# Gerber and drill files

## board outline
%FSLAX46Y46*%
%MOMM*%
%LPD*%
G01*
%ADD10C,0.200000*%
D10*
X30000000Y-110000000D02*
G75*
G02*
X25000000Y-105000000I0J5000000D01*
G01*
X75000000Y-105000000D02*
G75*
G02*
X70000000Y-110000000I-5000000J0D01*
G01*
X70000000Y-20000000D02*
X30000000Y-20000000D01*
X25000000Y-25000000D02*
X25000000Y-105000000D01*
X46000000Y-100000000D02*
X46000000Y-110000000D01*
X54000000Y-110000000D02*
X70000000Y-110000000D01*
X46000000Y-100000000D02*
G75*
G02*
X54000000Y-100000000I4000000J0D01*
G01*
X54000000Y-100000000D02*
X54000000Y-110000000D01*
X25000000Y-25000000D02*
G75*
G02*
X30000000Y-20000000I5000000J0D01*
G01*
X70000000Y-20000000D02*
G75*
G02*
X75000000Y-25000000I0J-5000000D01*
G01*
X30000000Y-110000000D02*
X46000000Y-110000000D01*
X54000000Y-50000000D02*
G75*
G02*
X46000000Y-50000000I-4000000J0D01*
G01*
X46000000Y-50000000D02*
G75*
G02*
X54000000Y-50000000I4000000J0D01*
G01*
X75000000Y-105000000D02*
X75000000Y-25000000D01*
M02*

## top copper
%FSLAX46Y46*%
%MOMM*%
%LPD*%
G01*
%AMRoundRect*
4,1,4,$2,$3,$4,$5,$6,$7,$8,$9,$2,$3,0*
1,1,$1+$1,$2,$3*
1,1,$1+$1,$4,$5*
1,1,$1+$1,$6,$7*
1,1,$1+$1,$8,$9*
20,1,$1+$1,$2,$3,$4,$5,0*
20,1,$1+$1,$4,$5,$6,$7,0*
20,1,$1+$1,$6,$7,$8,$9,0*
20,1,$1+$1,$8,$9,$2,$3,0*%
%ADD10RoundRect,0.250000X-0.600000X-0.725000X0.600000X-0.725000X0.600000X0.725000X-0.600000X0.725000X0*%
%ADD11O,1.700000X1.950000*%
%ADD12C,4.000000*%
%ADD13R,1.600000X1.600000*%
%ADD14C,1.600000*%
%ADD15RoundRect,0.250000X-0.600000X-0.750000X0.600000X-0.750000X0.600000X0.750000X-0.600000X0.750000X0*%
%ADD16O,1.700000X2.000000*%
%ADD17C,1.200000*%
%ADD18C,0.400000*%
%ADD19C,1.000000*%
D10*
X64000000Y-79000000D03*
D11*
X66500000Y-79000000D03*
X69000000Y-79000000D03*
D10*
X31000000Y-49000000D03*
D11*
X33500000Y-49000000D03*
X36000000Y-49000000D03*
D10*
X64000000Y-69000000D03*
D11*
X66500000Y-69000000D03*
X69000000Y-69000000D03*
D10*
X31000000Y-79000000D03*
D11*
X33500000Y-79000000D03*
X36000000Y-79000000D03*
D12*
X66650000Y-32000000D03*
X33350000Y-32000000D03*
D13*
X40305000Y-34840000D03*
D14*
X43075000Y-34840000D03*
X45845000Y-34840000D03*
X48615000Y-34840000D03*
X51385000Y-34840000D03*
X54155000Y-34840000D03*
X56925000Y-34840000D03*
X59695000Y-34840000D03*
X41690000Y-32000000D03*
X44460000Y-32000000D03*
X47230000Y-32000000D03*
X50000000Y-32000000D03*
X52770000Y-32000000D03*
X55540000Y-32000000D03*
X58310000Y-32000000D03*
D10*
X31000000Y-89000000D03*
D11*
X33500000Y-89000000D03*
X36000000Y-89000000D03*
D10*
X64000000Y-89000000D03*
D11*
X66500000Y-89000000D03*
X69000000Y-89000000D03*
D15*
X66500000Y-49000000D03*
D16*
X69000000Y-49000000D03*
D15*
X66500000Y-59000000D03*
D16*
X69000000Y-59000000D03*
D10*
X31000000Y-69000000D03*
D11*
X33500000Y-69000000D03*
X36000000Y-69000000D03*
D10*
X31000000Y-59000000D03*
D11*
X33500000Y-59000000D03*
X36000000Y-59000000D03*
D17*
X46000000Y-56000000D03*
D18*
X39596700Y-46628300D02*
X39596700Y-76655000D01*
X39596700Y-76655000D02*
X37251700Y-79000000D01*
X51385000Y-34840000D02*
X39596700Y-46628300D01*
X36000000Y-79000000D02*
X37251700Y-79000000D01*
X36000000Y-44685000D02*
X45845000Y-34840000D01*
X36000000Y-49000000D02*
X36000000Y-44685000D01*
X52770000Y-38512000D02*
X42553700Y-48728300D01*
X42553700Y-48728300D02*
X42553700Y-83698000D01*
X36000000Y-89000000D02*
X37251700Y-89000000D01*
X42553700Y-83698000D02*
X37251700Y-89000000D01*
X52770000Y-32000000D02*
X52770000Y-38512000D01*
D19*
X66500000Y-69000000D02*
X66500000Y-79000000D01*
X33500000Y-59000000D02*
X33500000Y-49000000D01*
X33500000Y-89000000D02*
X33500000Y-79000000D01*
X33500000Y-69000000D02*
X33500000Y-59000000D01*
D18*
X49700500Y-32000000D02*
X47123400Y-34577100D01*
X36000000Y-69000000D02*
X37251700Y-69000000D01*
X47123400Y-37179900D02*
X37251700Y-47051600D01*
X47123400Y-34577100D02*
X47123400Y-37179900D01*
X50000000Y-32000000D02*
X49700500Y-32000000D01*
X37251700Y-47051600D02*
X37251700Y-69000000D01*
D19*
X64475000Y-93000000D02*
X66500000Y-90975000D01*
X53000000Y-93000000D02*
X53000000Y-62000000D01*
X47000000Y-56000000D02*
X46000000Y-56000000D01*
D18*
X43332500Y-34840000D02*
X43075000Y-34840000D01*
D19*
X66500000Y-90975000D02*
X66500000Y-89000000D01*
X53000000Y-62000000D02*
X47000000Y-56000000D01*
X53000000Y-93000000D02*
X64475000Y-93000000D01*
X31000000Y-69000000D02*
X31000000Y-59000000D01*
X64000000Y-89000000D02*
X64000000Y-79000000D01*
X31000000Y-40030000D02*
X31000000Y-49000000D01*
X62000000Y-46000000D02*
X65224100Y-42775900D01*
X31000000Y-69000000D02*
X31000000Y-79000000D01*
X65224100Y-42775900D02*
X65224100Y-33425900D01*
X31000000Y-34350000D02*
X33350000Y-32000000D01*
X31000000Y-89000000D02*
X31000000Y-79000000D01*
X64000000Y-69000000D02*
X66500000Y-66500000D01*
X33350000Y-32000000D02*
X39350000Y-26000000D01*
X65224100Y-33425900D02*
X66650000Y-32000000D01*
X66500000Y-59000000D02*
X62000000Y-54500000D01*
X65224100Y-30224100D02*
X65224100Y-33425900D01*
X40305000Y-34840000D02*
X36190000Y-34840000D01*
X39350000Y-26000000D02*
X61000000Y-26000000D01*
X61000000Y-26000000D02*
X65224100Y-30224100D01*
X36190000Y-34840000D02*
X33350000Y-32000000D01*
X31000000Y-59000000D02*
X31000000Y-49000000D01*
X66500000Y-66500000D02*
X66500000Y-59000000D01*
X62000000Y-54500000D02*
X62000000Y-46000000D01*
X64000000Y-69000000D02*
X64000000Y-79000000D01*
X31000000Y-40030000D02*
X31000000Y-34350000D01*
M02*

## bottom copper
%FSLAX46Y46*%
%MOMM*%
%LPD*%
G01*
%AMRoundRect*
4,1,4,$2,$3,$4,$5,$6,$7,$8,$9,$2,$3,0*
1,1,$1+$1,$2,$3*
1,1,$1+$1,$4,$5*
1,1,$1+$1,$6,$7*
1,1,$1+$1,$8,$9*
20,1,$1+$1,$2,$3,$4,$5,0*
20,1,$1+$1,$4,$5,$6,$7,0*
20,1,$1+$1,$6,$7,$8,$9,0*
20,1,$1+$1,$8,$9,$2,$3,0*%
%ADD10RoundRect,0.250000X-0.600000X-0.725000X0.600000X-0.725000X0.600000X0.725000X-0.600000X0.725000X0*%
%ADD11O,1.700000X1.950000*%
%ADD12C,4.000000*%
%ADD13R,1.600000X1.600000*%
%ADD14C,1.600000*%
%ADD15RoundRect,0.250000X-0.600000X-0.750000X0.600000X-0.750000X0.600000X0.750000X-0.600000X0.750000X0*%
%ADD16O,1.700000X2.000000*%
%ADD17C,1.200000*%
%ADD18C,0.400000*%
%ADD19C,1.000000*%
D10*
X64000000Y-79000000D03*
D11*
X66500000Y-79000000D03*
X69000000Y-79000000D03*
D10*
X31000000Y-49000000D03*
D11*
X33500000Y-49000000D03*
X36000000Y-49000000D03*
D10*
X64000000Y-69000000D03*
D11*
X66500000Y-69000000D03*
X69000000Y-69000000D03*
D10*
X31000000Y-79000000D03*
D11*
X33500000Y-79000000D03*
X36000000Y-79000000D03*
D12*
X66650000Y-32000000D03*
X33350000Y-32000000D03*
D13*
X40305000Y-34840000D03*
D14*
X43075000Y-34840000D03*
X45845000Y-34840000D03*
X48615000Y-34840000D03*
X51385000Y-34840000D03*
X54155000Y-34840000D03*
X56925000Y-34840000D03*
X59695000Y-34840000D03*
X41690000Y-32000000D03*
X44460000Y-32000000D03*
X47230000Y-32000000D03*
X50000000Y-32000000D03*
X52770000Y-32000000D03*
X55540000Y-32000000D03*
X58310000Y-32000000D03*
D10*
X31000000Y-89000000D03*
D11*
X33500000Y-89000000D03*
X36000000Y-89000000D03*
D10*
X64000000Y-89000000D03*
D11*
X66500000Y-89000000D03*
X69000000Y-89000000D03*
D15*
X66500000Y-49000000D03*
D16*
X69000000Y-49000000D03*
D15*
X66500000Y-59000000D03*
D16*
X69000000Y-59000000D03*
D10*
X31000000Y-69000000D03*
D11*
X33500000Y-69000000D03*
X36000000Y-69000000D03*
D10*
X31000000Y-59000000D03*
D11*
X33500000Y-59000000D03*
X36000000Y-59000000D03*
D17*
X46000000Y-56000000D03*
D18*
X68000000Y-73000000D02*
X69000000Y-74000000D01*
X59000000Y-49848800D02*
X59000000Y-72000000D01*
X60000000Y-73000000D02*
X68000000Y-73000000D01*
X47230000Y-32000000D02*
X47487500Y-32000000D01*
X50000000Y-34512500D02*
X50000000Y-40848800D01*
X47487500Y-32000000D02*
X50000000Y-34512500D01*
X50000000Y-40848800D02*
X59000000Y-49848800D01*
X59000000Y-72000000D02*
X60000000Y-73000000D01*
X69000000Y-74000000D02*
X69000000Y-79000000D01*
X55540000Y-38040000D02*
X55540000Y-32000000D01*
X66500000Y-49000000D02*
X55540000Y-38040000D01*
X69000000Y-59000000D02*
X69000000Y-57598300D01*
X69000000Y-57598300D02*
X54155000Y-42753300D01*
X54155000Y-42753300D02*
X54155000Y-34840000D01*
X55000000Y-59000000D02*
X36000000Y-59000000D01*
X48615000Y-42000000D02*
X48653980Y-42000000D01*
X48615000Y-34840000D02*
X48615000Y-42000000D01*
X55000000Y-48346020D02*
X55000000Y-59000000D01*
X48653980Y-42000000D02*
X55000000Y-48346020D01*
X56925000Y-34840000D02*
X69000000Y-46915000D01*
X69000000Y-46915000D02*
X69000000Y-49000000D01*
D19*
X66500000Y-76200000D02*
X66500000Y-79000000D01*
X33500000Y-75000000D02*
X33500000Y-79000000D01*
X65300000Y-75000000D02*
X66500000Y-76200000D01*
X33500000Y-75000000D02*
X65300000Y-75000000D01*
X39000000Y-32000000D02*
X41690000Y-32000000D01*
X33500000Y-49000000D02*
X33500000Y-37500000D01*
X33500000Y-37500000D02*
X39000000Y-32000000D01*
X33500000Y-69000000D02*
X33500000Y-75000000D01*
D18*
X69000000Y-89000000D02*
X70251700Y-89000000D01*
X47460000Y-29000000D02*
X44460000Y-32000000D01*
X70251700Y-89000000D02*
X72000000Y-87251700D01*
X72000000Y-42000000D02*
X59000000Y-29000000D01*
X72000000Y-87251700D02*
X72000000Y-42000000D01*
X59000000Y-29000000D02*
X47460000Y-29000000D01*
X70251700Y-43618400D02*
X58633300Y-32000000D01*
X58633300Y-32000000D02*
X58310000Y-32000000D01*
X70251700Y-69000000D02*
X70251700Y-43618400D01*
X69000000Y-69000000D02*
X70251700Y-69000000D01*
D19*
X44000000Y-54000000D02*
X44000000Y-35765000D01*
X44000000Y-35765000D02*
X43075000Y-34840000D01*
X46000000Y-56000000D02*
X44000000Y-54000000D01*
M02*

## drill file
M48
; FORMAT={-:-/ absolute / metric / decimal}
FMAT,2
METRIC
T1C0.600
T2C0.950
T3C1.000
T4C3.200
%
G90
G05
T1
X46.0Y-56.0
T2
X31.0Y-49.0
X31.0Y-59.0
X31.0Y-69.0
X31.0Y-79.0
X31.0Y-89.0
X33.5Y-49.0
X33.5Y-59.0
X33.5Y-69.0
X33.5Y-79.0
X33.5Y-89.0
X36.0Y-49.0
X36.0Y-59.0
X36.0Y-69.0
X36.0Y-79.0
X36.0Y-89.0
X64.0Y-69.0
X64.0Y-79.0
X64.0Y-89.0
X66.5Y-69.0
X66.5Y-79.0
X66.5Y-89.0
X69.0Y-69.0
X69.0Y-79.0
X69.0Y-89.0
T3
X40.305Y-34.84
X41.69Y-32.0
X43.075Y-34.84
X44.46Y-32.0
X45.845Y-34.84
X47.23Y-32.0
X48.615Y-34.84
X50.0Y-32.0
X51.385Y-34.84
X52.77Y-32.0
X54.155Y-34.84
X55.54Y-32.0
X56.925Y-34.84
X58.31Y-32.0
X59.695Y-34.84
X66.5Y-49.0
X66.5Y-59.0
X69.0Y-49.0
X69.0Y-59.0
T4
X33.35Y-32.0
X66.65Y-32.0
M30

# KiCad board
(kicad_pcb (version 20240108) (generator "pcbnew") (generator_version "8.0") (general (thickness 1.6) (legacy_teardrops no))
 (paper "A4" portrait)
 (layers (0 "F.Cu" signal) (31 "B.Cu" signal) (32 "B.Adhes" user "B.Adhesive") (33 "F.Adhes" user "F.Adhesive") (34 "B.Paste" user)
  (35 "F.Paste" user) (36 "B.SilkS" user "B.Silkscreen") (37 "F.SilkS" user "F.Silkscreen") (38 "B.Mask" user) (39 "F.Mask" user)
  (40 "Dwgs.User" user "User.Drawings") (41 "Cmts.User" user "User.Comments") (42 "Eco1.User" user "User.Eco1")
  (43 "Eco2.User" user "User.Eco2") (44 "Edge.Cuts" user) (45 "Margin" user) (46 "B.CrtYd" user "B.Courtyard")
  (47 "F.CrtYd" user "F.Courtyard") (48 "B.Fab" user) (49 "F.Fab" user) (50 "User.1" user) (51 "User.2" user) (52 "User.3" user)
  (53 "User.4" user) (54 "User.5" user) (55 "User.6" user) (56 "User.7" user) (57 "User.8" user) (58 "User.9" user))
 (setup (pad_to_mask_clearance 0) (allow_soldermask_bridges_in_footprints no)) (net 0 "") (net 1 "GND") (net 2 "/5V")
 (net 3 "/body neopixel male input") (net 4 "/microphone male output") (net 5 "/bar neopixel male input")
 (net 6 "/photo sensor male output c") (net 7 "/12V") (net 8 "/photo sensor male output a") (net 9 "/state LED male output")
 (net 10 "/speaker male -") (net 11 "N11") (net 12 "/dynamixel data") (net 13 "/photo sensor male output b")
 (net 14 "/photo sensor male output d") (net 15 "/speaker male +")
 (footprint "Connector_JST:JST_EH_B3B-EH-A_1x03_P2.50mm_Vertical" (layer "F.Cu") (at 64 79)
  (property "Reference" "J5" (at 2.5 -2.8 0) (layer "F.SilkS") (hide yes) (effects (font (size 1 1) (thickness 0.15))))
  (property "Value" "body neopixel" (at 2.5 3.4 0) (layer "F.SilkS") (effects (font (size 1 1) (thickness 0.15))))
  (pad "1" thru_hole roundrect (at 0 0) (size 1.7 1.95) (drill 0.95) (layers "*.Cu" "*.Mask") (remove_unused_layers no)
   (roundrect_rratio 0.147059) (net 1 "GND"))
  (pad "2" thru_hole oval (at 2.5 0) (size 1.7 1.95) (drill 0.95) (layers "*.Cu" "*.Mask") (remove_unused_layers no) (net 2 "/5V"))
  (pad "3" thru_hole oval (at 5 0) (size 1.7 1.95) (drill 0.95) (layers "*.Cu" "*.Mask") (remove_unused_layers no)
   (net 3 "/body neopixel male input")))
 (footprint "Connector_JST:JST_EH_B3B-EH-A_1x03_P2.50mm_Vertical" (layer "F.Cu") (at 31 49)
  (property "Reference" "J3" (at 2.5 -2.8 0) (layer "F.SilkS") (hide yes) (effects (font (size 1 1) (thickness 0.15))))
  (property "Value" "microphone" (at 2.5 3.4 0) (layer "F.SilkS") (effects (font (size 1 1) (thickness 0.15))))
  (pad "1" thru_hole roundrect (at 0 0) (size 1.7 1.95) (drill 0.95) (layers "*.Cu" "*.Mask") (remove_unused_layers no)
   (roundrect_rratio 0.147059) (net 1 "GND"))
  (pad "2" thru_hole oval (at 2.5 0) (size 1.7 1.95) (drill 0.95) (layers "*.Cu" "*.Mask") (remove_unused_layers no) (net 2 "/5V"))
  (pad "3" thru_hole oval (at 5 0) (size 1.7 1.95) (drill 0.95) (layers "*.Cu" "*.Mask") (remove_unused_layers no)
   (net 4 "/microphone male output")))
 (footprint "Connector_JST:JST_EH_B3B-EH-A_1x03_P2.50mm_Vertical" (layer "F.Cu") (at 64 69)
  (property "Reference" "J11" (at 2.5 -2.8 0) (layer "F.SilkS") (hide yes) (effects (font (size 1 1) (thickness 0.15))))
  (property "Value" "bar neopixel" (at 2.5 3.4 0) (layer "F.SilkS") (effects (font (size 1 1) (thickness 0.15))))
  (pad "1" thru_hole roundrect (at 0 0) (size 1.7 1.95) (drill 0.95) (layers "*.Cu" "*.Mask") (remove_unused_layers no)
   (roundrect_rratio 0.147059) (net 1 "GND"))
  (pad "2" thru_hole oval (at 2.5 0) (size 1.7 1.95) (drill 0.95) (layers "*.Cu" "*.Mask") (remove_unused_layers no) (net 2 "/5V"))
  (pad "3" thru_hole oval (at 5 0) (size 1.7 1.95) (drill 0.95) (layers "*.Cu" "*.Mask") (remove_unused_layers no)
   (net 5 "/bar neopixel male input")))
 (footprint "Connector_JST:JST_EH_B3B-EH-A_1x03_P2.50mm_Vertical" (layer "F.Cu") (at 31 79)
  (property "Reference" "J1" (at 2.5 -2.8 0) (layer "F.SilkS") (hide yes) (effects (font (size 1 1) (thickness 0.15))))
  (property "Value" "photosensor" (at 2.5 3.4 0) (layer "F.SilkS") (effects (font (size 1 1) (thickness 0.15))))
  (pad "1" thru_hole roundrect (at 0 0) (size 1.7 1.95) (drill 0.95) (layers "*.Cu" "*.Mask") (remove_unused_layers no)
   (roundrect_rratio 0.147059) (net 1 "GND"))
  (pad "2" thru_hole oval (at 2.5 0) (size 1.7 1.95) (drill 0.95) (layers "*.Cu" "*.Mask") (remove_unused_layers no) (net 2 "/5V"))
  (pad "3" thru_hole oval (at 5 0) (size 1.7 1.95) (drill 0.95) (layers "*.Cu" "*.Mask") (remove_unused_layers no)
   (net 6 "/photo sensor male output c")))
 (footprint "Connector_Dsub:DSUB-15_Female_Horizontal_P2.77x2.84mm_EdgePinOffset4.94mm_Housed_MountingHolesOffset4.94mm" (layer "F.Cu")
  (at 40.305 34.84 180)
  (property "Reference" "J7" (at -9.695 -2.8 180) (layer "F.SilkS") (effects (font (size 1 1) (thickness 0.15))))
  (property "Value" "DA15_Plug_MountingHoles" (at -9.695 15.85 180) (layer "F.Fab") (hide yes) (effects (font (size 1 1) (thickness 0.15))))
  (pad "0" thru_hole circle (at -26.345 2.84 180) (size 4 4) (drill 3.2) (layers "*.Cu" "*.Mask") (remove_unused_layers no) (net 1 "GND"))
  (pad "0" thru_hole circle (at 6.955 2.84 180) (size 4 4) (drill 3.2) (layers "*.Cu" "*.Mask") (remove_unused_layers no) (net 1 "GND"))
  (pad "1" thru_hole rect (at 0 0 180) (size 1.6 1.6) (drill 1) (layers "*.Cu" "*.Mask") (remove_unused_layers no) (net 1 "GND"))
  (pad "2" thru_hole circle (at -2.77 0 180) (size 1.6 1.6) (drill 1) (layers "*.Cu" "*.Mask") (remove_unused_layers no) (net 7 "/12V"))
  (pad "3" thru_hole circle (at -5.54 0 180) (size 1.6 1.6) (drill 1) (layers "*.Cu" "*.Mask") (remove_unused_layers no)
   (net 4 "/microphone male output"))
  (pad "4" thru_hole circle (at -8.31 0 180) (size 1.6 1.6) (drill 1) (layers "*.Cu" "*.Mask") (remove_unused_layers no)
   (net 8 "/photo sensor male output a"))
  (pad "5" thru_hole circle (at -11.08 0 180) (size 1.6 1.6) (drill 1) (layers "*.Cu" "*.Mask") (remove_unused_layers no)
   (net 6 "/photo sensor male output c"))
  (pad "6" thru_hole circle (at -13.85 0 180) (size 1.6 1.6) (drill 1) (layers "*.Cu" "*.Mask") (remove_unused_layers no)
   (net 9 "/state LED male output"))
  (pad "7" thru_hole circle (at -16.62 0 180) (size 1.6 1.6) (drill 1) (layers "*.Cu" "*.Mask") (remove_unused_layers no)
   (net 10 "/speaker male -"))
  (pad "8" thru_hole circle (at -19.39 0 180) (size 1.6 1.6) (drill 1) (layers "*.Cu" "*.Mask") (remove_unused_layers no) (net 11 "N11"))
  (pad "9" thru_hole circle (at -1.385 2.84 180) (size 1.6 1.6) (drill 1) (layers "*.Cu" "*.Mask") (remove_unused_layers no) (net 2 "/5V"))
  (pad "10" thru_hole circle (at -4.155 2.84 180) (size 1.6 1.6) (drill 1) (layers "*.Cu" "*.Mask") (remove_unused_layers no)
   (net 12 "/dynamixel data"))
  (pad "11" thru_hole circle (at -6.925 2.84 180) (size 1.6 1.6) (drill 1) (layers "*.Cu" "*.Mask") (remove_unused_layers no)
   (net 3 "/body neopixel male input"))
  (pad "12" thru_hole circle (at -9.695 2.84 180) (size 1.6 1.6) (drill 1) (layers "*.Cu" "*.Mask") (remove_unused_layers no)
   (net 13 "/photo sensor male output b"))
  (pad "13" thru_hole circle (at -12.465 2.84 180) (size 1.6 1.6) (drill 1) (layers "*.Cu" "*.Mask") (remove_unused_layers no)
   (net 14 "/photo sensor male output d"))
  (pad "14" thru_hole circle (at -15.235 2.84 180) (size 1.6 1.6) (drill 1) (layers "*.Cu" "*.Mask") (remove_unused_layers no)
   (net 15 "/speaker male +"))
  (pad "15" thru_hole circle (at -18.005 2.84 180) (size 1.6 1.6) (drill 1) (layers "*.Cu" "*.Mask") (remove_unused_layers no)
   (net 5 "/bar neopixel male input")))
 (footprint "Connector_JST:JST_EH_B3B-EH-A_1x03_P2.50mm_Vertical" (layer "F.Cu") (at 31 89)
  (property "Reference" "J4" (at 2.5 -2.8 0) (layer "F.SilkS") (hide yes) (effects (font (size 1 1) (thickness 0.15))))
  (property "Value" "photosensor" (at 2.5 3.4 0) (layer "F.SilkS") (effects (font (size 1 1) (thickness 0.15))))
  (pad "1" thru_hole roundrect (at 0 0) (size 1.7 1.95) (drill 0.95) (layers "*.Cu" "*.Mask") (remove_unused_layers no)
   (roundrect_rratio 0.147059) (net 1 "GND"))
  (pad "2" thru_hole oval (at 2.5 0) (size 1.7 1.95) (drill 0.95) (layers "*.Cu" "*.Mask") (remove_unused_layers no) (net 2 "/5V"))
  (pad "3" thru_hole oval (at 5 0) (size 1.7 1.95) (drill 0.95) (layers "*.Cu" "*.Mask") (remove_unused_layers no)
   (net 14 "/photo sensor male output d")))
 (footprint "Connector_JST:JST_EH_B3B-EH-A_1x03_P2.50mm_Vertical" (layer "F.Cu") (at 64 89)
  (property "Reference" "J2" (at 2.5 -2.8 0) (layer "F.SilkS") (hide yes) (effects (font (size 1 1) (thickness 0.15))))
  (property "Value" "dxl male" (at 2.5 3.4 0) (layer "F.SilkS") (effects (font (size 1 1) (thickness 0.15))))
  (pad "1" thru_hole roundrect (at 0 0) (size 1.7 1.95) (drill 0.95) (layers "*.Cu" "*.Mask") (remove_unused_layers no)
   (roundrect_rratio 0.147059) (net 1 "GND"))
  (pad "2" thru_hole oval (at 2.5 0) (size 1.7 1.95) (drill 0.95) (layers "*.Cu" "*.Mask") (remove_unused_layers no) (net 7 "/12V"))
  (pad "3" thru_hole oval (at 5 0) (size 1.7 1.95) (drill 0.95) (layers "*.Cu" "*.Mask") (remove_unused_layers no)
   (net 12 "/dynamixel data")))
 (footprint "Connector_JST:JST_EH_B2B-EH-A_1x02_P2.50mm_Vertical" (layer "F.Cu") (at 66.5 49)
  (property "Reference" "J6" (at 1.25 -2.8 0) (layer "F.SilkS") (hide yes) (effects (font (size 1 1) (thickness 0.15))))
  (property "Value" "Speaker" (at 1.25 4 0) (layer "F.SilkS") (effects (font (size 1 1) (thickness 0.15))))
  (pad "1" thru_hole roundrect (at 0 0) (size 1.7 2) (drill 1) (layers "*.Cu" "*.Mask") (remove_unused_layers no)
   (roundrect_rratio 0.147059) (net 15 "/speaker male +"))
  (pad "2" thru_hole oval (at 2.5 0) (size 1.7 2) (drill 1) (layers "*.Cu" "*.Mask") (remove_unused_layers no) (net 10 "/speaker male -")))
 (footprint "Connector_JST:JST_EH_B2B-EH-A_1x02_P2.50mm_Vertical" (layer "F.Cu") (at 66.5 59)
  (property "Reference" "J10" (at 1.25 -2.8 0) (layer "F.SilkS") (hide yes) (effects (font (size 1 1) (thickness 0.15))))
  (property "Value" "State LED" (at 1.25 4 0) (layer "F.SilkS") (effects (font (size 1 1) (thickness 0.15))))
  (pad "1" thru_hole roundrect (at 0 0) (size 1.7 2) (drill 1) (layers "*.Cu" "*.Mask") (remove_unused_layers no)
   (roundrect_rratio 0.147059) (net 1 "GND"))
  (pad "2" thru_hole oval (at 2.5 0) (size 1.7 2) (drill 1) (layers "*.Cu" "*.Mask") (remove_unused_layers no)
   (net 9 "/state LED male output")))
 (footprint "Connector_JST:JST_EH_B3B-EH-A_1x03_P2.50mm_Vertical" (layer "F.Cu") (at 31 69)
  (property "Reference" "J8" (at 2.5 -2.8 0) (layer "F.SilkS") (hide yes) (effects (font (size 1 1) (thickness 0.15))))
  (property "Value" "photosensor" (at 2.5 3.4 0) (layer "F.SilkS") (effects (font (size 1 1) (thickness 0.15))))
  (pad "1" thru_hole roundrect (at 0 0) (size 1.7 1.95) (drill 0.95) (layers "*.Cu" "*.Mask") (remove_unused_layers no)
   (roundrect_rratio 0.147059) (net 1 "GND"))
  (pad "2" thru_hole oval (at 2.5 0) (size 1.7 1.95) (drill 0.95) (layers "*.Cu" "*.Mask") (remove_unused_layers no) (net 2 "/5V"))
  (pad "3" thru_hole oval (at 5 0) (size 1.7 1.95) (drill 0.95) (layers "*.Cu" "*.Mask") (remove_unused_layers no)
   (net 13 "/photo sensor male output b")))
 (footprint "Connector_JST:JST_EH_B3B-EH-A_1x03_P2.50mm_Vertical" (layer "F.Cu") (at 31 59)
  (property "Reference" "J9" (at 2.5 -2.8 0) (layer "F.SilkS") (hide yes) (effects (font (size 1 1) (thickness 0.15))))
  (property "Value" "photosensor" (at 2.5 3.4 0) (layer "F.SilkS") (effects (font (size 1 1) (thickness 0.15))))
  (pad "1" thru_hole roundrect (at 0 0) (size 1.7 1.95) (drill 0.95) (layers "*.Cu" "*.Mask") (remove_unused_layers no)
   (roundrect_rratio 0.147059) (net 1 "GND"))
  (pad "2" thru_hole oval (at 2.5 0) (size 1.7 1.95) (drill 0.95) (layers "*.Cu" "*.Mask") (remove_unused_layers no) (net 2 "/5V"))
  (pad "3" thru_hole oval (at 5 0) (size 1.7 1.95) (drill 0.95) (layers "*.Cu" "*.Mask") (remove_unused_layers no)
   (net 8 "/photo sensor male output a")))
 (gr_arc (start 30 110) (mid 26.464466 108.535534) (end 25 105) (stroke (width 0.2) (type default)) (layer "Edge.Cuts"))
 (gr_arc (start 75 105) (mid 73.535534 108.535534) (end 70 110) (stroke (width 0.2) (type default)) (layer "Edge.Cuts"))
 (gr_line (start 70 20) (end 30 20) (stroke (width 0.2) (type default)) (layer "Edge.Cuts"))
 (gr_line (start 25 25) (end 25 105) (stroke (width 0.2) (type default)) (layer "Edge.Cuts"))
 (gr_line (start 46 100) (end 46 110) (stroke (width 0.2) (type default)) (layer "Edge.Cuts"))
 (gr_line (start 54 110) (end 70 110) (stroke (width 0.2) (type default)) (layer "Edge.Cuts"))
 (gr_arc (start 46 100) (mid 50 96) (end 54 100) (stroke (width 0.2) (type default)) (layer "Edge.Cuts"))
 (gr_line (start 54 100) (end 54 110) (stroke (width 0.2) (type default)) (layer "Edge.Cuts"))
 (gr_arc (start 25 25) (mid 26.464466 21.464466) (end 30 20) (stroke (width 0.2) (type default)) (layer "Edge.Cuts"))
 (gr_arc (start 70 20) (mid 73.535534 21.464466) (end 75 25) (stroke (width 0.2) (type default)) (layer "Edge.Cuts"))
 (gr_line (start 30 110) (end 46 110) (stroke (width 0.2) (type default)) (layer "Edge.Cuts"))
 (gr_circle (center 50 50) (end 54 50) (stroke (width 0.2) (type default)) (fill none) (layer "Edge.Cuts"))
 (gr_line (start 75 105) (end 75 25) (stroke (width 0.2) (type default)) (layer "Edge.Cuts"))
 (segment (start 39.5967 46.6283) (end 39.5967 76.655) (width 0.4) (layer "F.Cu") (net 6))
 (segment (start 39.5967 76.655) (end 37.2517 79) (width 0.4) (layer "F.Cu") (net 6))
 (segment (start 51.385 34.84) (end 39.5967 46.6283) (width 0.4) (layer "F.Cu") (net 6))
 (segment (start 36 79) (end 37.2517 79) (width 0.4) (layer "F.Cu") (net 6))
 (segment (start 36 44.685) (end 45.845 34.84) (width 0.4) (layer "F.Cu") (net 4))
 (segment (start 36 49) (end 36 44.685) (width 0.4) (layer "F.Cu") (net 4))
 (segment (start 52.77 38.512) (end 42.5537 48.7283) (width 0.4) (layer "F.Cu") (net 14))
 (segment (start 42.5537 48.7283) (end 42.5537 83.698) (width 0.4) (layer "F.Cu") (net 14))
 (segment (start 36 89) (end 37.2517 89) (width 0.4) (layer "F.Cu") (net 14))
 (segment (start 42.5537 83.698) (end 37.2517 89) (width 0.4) (layer "F.Cu") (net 14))
 (segment (start 52.77 32) (end 52.77 38.512) (width 0.4) (layer "F.Cu") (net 14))
 (segment (start 68 73) (end 69 74) (width 0.4) (layer "B.Cu") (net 3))
 (segment (start 59 49.8488) (end 59 72) (width 0.4) (layer "B.Cu") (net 3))
 (segment (start 60 73) (end 68 73) (width 0.4) (layer "B.Cu") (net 3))
 (segment (start 47.23 32) (end 47.4875 32) (width 0.4) (layer "B.Cu") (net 3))
 (segment (start 50 34.5125) (end 50 40.8488) (width 0.4) (layer "B.Cu") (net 3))
 (segment (start 47.4875 32) (end 50 34.5125) (width 0.4) (layer "B.Cu") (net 3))
 (segment (start 50 40.8488) (end 59 49.8488) (width 0.4) (layer "B.Cu") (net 3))
 (segment (start 59 72) (end 60 73) (width 0.4) (layer "B.Cu") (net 3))
 (segment (start 69 74) (end 69 79) (width 0.4) (layer "B.Cu") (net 3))
 (segment (start 55.54 38.04) (end 55.54 32) (width 0.4) (layer "B.Cu") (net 15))
 (segment (start 66.5 49) (end 55.54 38.04) (width 0.4) (layer "B.Cu") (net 15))
 (segment (start 69 59) (end 69 57.5983) (width 0.4) (layer "B.Cu") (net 9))
 (segment (start 69 57.5983) (end 54.155 42.7533) (width 0.4) (layer "B.Cu") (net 9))
 (segment (start 54.155 42.7533) (end 54.155 34.84) (width 0.4) (layer "B.Cu") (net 9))
 (segment (start 55 59) (end 36 59) (width 0.4) (layer "B.Cu") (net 8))
 (segment (start 48.615 42) (end 48.65398 42) (width 0.4) (layer "B.Cu") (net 8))
 (segment (start 48.615 34.84) (end 48.615 42) (width 0.4) (layer "B.Cu") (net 8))
 (segment (start 55 48.34602) (end 55 59) (width 0.4) (layer "B.Cu") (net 8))
 (segment (start 48.65398 42) (end 55 48.34602) (width 0.4) (layer "B.Cu") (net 8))
 (segment (start 56.925 34.84) (end 69 46.915) (width 0.4) (layer "B.Cu") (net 10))
 (segment (start 69 46.915) (end 69 49) (width 0.4) (layer "B.Cu") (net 10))
 (segment (start 66.5 69) (end 66.5 79) (width 1) (layer "F.Cu") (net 2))
 (segment (start 33.5 59) (end 33.5 49) (width 1) (layer "F.Cu") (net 2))
 (segment (start 33.5 89) (end 33.5 79) (width 1) (layer "F.Cu") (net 2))
 (segment (start 33.5 69) (end 33.5 59) (width 1) (layer "F.Cu") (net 2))
 (segment (start 66.5 76.2) (end 66.5 79) (width 1) (layer "B.Cu") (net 2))
 (segment (start 33.5 75) (end 33.5 79) (width 1) (layer "B.Cu") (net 2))
 (segment (start 65.3 75) (end 66.5 76.2) (width 1) (layer "B.Cu") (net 2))
 (segment (start 33.5 75) (end 65.3 75) (width 1) (layer "B.Cu") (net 2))
 (segment (start 39 32) (end 41.69 32) (width 1) (layer "B.Cu") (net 2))
 (segment (start 33.5 49) (end 33.5 37.5) (width 1) (layer "B.Cu") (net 2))
 (segment (start 33.5 37.5) (end 39 32) (width 1) (layer "B.Cu") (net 2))
 (segment (start 33.5 69) (end 33.5 75) (width 1) (layer "B.Cu") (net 2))
 (segment (start 49.7005 32) (end 47.1234 34.5771) (width 0.4) (layer "F.Cu") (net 13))
 (segment (start 36 69) (end 37.2517 69) (width 0.4) (layer "F.Cu") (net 13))
 (segment (start 47.1234 37.1799) (end 37.2517 47.0516) (width 0.4) (layer "F.Cu") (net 13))
 (segment (start 47.1234 34.5771) (end 47.1234 37.1799) (width 0.4) (layer "F.Cu") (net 13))
 (segment (start 50 32) (end 49.7005 32) (width 0.4) (layer "F.Cu") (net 13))
 (segment (start 37.2517 47.0516) (end 37.2517 69) (width 0.4) (layer "F.Cu") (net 13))
 (segment (start 69 89) (end 70.2517 89) (width 0.4) (layer "B.Cu") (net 12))
 (segment (start 47.46 29) (end 44.46 32) (width 0.4) (layer "B.Cu") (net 12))
 (segment (start 70.2517 89) (end 72 87.2517) (width 0.4) (layer "B.Cu") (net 12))
 (segment (start 72 42) (end 59 29) (width 0.4) (layer "B.Cu") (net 12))
 (segment (start 72 87.2517) (end 72 42) (width 0.4) (layer "B.Cu") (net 12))
 (segment (start 59 29) (end 47.46 29) (width 0.4) (layer "B.Cu") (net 12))
 (segment (start 70.2517 43.6184) (end 58.6333 32) (width 0.4) (layer "B.Cu") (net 5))
 (segment (start 58.6333 32) (end 58.31 32) (width 0.4) (layer "B.Cu") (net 5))
 (segment (start 70.2517 69) (end 70.2517 43.6184) (width 0.4) (layer "B.Cu") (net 5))
 (segment (start 69 69) (end 70.2517 69) (width 0.4) (layer "B.Cu") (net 5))
 (segment (start 64.475 93) (end 66.5 90.975) (width 1) (layer "F.Cu") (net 7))
 (segment (start 53 93) (end 53 62) (width 1) (layer "F.Cu") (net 7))
 (segment (start 47 56) (end 46 56) (width 1) (layer "F.Cu") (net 7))
 (segment (start 43.3325 34.84) (end 43.075 34.84) (width 0.4) (layer "F.Cu") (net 7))
 (segment (start 66.5 90.975) (end 66.5 89) (width 1) (layer "F.Cu") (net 7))
 (segment (start 53 62) (end 47 56) (width 1) (layer "F.Cu") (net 7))
 (segment (start 53 93) (end 64.475 93) (width 1) (layer "F.Cu") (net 7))
 (via (at 46 56) (size 1.2) (drill 0.6) (layers "F.Cu" "B.Cu") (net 7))
 (segment (start 44 54) (end 44 35.765) (width 1) (layer "B.Cu") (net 7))
 (segment (start 44 35.765) (end 43.075 34.84) (width 1) (layer "B.Cu") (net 7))
 (segment (start 46 56) (end 44 54) (width 1) (layer "B.Cu") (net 7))
 (segment (start 31 69) (end 31 59) (width 1) (layer "F.Cu") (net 1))
 (segment (start 64 89) (end 64 79) (width 1) (layer "F.Cu") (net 1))
 (segment (start 31 40.03) (end 31 49) (width 1) (layer "F.Cu") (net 1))
 (segment (start 62 46) (end 65.2241 42.7759) (width 1) (layer "F.Cu") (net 1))
 (segment (start 31 69) (end 31 79) (width 1) (layer "F.Cu") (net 1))
 (segment (start 65.2241 42.7759) (end 65.2241 33.4259) (width 1) (layer "F.Cu") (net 1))
 (segment (start 31 34.35) (end 33.35 32) (width 1) (layer "F.Cu") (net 1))
 (segment (start 31 89) (end 31 79) (width 1) (layer "F.Cu") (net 1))
 (segment (start 64 69) (end 66.5 66.5) (width 1) (layer "F.Cu") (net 1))
 (segment (start 33.35 32) (end 39.35 26) (width 1) (layer "F.Cu") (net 1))
 (segment (start 65.2241 33.4259) (end 66.65 32) (width 1) (layer "F.Cu") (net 1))
 (segment (start 66.5 59) (end 62 54.5) (width 1) (layer "F.Cu") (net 1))
 (segment (start 65.2241 30.2241) (end 65.2241 33.4259) (width 1) (layer "F.Cu") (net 1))
 (segment (start 40.305 34.84) (end 36.19 34.84) (width 1) (layer "F.Cu") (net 1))
 (segment (start 39.35 26) (end 61 26) (width 1) (layer "F.Cu") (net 1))
 (segment (start 61 26) (end 65.2241 30.2241) (width 1) (layer "F.Cu") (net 1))
 (segment (start 36.19 34.84) (end 33.35 32) (width 1) (layer "F.Cu") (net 1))
 (segment (start 31 59) (end 31 49) (width 1) (layer "F.Cu") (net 1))
 (segment (start 66.5 66.5) (end 66.5 59) (width 1) (layer "F.Cu") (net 1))
 (segment (start 62 54.5) (end 62 46) (width 1) (layer "F.Cu") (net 1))
 (segment (start 64 69) (end 64 79) (width 1) (layer "F.Cu") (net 1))
 (segment (start 31 40.03) (end 31 34.35) (width 1) (layer "F.Cu") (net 1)))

